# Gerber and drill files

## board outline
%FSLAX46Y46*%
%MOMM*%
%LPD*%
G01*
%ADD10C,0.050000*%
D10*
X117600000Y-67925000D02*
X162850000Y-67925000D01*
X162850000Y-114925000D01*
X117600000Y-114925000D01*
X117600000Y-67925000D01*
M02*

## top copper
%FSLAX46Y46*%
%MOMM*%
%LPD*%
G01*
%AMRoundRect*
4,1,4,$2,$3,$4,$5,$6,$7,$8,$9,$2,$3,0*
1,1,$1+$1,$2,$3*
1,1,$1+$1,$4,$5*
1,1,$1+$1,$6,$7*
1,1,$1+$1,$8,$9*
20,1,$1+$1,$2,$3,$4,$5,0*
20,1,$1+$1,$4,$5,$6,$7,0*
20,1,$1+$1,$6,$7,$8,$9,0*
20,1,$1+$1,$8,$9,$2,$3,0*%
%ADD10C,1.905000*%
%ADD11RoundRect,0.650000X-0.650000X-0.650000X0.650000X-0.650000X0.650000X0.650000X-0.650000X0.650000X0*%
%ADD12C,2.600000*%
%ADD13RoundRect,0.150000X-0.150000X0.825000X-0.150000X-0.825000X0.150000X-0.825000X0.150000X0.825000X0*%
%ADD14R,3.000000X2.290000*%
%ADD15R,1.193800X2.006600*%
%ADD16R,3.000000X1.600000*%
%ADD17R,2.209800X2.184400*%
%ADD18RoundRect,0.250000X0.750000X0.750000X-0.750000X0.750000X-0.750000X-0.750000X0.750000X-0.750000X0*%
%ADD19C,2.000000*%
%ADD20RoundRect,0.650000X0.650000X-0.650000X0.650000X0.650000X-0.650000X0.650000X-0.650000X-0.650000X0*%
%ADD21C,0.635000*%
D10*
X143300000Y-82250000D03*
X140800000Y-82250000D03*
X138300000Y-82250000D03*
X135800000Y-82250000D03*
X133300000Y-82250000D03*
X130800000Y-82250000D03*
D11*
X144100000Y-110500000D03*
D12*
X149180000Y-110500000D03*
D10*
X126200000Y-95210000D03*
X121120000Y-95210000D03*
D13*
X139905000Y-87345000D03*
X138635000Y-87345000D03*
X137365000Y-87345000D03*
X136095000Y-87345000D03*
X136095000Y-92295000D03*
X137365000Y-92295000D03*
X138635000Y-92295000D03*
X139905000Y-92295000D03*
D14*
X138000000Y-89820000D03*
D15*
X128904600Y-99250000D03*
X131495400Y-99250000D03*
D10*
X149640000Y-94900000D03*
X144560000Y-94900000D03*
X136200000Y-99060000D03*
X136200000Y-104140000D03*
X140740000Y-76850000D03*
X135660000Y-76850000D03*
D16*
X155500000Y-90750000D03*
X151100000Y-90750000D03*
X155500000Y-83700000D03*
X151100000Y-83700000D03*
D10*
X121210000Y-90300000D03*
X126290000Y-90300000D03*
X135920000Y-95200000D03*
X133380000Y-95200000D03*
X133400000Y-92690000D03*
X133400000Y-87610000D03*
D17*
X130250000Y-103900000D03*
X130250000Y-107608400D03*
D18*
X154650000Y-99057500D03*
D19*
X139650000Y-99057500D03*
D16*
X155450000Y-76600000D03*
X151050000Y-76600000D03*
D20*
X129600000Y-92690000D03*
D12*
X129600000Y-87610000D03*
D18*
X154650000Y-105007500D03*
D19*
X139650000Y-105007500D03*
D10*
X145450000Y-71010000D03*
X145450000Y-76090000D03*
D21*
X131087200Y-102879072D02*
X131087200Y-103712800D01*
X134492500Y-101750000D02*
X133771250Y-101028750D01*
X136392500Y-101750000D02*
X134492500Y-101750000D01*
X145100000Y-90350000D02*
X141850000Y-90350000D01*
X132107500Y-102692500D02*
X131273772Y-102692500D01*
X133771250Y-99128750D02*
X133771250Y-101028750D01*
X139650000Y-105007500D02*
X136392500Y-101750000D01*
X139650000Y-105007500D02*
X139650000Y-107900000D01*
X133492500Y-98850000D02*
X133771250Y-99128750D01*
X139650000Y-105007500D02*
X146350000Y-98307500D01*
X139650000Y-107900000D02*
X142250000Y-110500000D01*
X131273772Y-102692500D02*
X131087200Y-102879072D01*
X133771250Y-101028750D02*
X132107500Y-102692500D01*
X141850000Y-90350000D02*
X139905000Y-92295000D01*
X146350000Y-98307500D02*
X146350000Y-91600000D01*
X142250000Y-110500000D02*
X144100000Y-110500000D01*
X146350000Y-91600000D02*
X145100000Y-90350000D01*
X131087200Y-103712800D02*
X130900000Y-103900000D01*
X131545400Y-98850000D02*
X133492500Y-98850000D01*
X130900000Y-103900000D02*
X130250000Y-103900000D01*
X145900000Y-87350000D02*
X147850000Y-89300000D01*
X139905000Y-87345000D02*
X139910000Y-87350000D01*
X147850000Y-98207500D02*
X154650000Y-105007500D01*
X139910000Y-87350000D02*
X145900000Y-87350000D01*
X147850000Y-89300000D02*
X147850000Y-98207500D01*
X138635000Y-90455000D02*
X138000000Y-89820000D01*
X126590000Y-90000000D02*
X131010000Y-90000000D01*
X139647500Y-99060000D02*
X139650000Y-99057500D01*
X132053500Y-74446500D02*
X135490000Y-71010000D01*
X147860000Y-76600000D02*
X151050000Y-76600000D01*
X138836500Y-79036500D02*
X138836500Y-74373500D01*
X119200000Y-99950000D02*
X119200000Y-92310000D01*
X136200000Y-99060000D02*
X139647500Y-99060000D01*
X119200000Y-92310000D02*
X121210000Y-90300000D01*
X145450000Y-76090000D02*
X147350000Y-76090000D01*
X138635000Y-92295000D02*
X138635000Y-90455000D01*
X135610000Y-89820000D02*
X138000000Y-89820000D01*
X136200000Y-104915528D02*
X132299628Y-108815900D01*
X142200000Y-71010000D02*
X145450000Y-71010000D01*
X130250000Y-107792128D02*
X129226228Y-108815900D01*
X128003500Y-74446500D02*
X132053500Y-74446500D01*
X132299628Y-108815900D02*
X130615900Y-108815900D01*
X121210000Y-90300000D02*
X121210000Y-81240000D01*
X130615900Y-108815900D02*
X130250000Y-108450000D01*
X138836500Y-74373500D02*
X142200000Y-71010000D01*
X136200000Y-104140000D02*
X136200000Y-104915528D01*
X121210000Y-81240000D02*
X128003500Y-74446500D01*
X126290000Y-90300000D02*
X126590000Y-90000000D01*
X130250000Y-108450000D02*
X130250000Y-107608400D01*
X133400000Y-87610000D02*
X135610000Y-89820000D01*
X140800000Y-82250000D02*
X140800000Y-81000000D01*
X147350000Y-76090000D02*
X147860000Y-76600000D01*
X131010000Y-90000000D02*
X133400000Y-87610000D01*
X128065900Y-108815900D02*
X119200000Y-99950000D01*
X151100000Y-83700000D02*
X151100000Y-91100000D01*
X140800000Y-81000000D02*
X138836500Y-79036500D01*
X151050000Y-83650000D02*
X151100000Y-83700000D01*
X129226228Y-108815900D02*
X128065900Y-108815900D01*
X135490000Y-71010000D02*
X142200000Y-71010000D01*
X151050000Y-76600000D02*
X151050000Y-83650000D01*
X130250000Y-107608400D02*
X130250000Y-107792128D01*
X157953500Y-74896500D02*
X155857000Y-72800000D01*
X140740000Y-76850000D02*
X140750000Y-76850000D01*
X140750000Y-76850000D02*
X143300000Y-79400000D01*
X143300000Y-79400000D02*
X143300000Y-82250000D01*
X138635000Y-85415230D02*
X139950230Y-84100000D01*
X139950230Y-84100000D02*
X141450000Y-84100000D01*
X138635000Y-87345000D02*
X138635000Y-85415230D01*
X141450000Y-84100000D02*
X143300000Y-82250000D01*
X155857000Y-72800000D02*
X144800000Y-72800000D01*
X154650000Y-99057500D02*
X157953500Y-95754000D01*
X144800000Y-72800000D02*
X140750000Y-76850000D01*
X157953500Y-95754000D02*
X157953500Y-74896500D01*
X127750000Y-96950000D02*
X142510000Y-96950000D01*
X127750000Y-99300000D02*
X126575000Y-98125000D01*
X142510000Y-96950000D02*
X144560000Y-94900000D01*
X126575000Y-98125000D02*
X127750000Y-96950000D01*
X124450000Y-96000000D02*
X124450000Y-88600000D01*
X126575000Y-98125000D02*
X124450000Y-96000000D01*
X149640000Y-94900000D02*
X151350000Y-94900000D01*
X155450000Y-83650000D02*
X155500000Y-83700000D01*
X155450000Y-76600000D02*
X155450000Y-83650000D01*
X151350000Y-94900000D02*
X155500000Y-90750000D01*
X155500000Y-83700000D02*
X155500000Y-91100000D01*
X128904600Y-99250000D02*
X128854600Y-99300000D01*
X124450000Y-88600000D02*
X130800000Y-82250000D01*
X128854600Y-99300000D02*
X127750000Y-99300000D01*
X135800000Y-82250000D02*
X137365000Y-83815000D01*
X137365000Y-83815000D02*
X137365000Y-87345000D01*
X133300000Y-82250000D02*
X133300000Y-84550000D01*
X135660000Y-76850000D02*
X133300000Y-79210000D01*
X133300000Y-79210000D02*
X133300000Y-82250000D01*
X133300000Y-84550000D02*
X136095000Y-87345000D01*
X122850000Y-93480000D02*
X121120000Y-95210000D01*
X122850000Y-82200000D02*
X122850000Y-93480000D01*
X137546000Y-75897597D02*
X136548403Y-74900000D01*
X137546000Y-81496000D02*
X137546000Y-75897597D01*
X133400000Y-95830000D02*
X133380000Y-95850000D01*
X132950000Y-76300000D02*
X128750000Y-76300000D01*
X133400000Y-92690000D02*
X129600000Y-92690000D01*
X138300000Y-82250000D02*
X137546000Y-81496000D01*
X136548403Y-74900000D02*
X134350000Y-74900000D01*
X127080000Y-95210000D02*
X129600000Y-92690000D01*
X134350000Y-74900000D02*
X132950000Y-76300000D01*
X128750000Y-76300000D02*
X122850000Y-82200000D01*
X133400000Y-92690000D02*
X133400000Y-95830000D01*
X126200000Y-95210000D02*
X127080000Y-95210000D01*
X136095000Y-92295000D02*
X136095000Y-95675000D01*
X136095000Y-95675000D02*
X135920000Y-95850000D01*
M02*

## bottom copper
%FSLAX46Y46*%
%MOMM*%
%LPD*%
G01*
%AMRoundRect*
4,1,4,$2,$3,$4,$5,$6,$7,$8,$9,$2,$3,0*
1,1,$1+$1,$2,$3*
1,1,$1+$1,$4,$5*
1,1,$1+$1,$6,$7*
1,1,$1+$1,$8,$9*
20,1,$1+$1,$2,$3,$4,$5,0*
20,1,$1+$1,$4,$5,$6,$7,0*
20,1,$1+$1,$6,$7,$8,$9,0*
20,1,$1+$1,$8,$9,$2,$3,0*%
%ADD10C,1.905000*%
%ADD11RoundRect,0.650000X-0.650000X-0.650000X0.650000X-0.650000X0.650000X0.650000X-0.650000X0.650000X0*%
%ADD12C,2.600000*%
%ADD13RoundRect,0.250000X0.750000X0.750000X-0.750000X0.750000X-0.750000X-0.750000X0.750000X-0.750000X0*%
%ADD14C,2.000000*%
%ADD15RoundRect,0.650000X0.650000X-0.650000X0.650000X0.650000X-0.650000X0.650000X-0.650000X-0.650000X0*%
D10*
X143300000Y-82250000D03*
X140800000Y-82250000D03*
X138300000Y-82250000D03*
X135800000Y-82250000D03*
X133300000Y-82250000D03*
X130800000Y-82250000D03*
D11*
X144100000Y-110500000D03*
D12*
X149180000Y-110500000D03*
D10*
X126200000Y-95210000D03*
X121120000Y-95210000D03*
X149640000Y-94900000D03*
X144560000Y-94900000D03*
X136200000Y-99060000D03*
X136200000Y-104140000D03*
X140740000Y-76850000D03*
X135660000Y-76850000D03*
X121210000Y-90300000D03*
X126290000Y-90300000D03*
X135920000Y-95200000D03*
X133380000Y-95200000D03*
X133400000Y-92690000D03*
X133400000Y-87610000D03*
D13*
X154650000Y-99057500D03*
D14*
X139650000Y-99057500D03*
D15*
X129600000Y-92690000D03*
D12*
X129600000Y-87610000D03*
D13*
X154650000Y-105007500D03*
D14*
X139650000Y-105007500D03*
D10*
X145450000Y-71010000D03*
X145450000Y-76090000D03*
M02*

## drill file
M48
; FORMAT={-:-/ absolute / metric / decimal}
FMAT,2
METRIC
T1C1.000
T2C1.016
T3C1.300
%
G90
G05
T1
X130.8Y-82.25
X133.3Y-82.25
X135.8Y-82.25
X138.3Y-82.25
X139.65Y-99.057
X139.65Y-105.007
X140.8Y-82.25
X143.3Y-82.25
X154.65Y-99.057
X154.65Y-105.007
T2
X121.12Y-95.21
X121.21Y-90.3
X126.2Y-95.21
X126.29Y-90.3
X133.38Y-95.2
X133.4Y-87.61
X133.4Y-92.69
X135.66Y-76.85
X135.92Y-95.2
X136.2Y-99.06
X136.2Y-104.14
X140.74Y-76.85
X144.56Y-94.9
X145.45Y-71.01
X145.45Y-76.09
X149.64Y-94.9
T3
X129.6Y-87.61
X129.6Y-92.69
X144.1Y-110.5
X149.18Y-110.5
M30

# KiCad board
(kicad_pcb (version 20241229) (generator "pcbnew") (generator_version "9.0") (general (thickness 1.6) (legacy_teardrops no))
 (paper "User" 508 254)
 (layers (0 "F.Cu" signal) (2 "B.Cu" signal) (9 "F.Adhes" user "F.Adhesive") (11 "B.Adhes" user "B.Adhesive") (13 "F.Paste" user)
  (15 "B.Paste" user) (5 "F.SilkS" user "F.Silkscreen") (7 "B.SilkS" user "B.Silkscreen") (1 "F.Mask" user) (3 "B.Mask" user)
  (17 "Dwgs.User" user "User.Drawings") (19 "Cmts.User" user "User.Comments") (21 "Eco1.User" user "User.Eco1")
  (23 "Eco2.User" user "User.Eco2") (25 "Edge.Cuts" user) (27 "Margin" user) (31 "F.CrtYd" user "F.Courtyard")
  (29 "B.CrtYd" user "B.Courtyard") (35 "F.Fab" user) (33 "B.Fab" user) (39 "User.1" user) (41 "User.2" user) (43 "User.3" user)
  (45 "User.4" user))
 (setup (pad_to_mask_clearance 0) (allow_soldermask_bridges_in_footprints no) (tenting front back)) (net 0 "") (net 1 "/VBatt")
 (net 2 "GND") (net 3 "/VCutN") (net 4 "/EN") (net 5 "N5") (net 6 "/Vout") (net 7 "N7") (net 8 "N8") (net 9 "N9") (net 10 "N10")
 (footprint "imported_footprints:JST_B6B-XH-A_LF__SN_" (layer "F.Cu") (at 137.05 81.725)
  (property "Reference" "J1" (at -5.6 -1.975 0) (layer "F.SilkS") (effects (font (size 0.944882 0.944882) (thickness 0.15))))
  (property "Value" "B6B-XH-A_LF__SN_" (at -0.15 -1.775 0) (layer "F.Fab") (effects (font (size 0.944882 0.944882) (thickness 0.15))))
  (pad "1" thru_hole circle (at 6.25 0.525) (size 1.905 1.905) (drill 1) (layers "*.Cu" "*.Mask") (remove_unused_layers no) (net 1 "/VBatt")
   (solder_mask_margin 0.102))
  (pad "2" thru_hole circle (at 3.75 0.525) (size 1.905 1.905) (drill 1) (layers "*.Cu" "*.Mask") (remove_unused_layers no) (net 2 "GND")
   (solder_mask_margin 0.102))
  (pad "3" thru_hole circle (at 1.25 0.525) (size 1.905 1.905) (drill 1) (layers "*.Cu" "*.Mask") (remove_unused_layers no) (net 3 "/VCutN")
   (solder_mask_margin 0.102))
  (pad "4" thru_hole circle (at -1.25 0.525) (size 1.905 1.905) (drill 1) (layers "*.Cu" "*.Mask") (remove_unused_layers no) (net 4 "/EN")
   (solder_mask_margin 0.102))
  (pad "5" thru_hole circle (at -3.75 0.525) (size 1.905 1.905) (drill 1) (layers "*.Cu" "*.Mask") (remove_unused_layers no) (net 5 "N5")
   (solder_mask_margin 0.102))
  (pad "6" thru_hole circle (at -6.25 0.525) (size 1.905 1.905) (drill 1) (layers "*.Cu" "*.Mask") (remove_unused_layers no) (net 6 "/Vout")
   (solder_mask_margin 0.102)))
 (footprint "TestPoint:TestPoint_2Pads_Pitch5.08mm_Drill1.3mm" (layer "F.Cu") (at 144.1 110.5)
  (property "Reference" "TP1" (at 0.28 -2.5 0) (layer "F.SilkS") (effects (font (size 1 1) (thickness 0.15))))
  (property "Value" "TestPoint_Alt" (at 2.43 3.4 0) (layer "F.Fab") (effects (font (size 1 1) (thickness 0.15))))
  (pad "1" thru_hole roundrect (at 0 0) (size 2.6 2.6) (drill 1.3) (layers "*.Cu" "*.Mask") (remove_unused_layers no)
   (roundrect_rratio 0.25) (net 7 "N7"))
  (pad "2" thru_hole circle (at 5.08 0) (size 2.6 2.6) (drill 1.3) (layers "*.Cu" "*.Mask") (remove_unused_layers no)))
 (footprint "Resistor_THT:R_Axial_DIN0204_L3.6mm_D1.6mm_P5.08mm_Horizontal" (layer "F.Cu") (at 126.2 95.21 180)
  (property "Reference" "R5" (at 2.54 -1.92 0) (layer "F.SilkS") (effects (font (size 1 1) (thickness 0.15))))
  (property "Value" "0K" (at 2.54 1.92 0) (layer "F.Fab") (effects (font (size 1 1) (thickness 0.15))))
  (pad "1" thru_hole circle (at 0 0 180) (size 1.905 1.905) (drill 1.016) (layers "*.Cu" "*.Mask") (remove_unused_layers no)
   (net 3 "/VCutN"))
  (pad "2" thru_hole circle (at 5.08 0 180) (size 1.905 1.905) (drill 1.016) (layers "*.Cu" "*.Mask") (remove_unused_layers no)
   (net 3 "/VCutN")))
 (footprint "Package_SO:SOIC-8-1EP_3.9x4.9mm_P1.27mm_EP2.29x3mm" (layer "F.Cu") (at 138 89.82 -90)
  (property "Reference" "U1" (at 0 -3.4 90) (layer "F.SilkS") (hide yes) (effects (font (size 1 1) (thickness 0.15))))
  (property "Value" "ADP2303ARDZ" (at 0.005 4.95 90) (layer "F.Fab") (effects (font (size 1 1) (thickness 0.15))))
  (pad "" smd roundrect (at -0.57 -0.75 270) (size 0.92 1.21) (layers "F.Paste") (roundrect_rratio 0.25))
  (pad "" smd roundrect (at -0.57 0.75 270) (size 0.92 1.21) (layers "F.Paste") (roundrect_rratio 0.25))
  (pad "" smd roundrect (at 0.57 -0.75 270) (size 0.92 1.21) (layers "F.Paste") (roundrect_rratio 0.25))
  (pad "" smd roundrect (at 0.57 0.75 270) (size 0.92 1.21) (layers "F.Paste") (roundrect_rratio 0.25))
  (pad "1" smd roundrect (at -2.475 -1.905 270) (size 1.95 0.6) (layers "F.Cu" "F.Mask" "F.Paste") (roundrect_rratio 0.25) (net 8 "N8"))
  (pad "2" smd roundrect (at -2.475 -0.635 270) (size 1.95 0.6) (layers "F.Cu" "F.Mask" "F.Paste") (roundrect_rratio 0.25) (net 1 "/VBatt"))
  (pad "3" smd roundrect (at -2.475 0.635 270) (size 1.95 0.6) (layers "F.Cu" "F.Mask" "F.Paste") (roundrect_rratio 0.25) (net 4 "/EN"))
  (pad "4" smd roundrect (at -2.475 1.905 270) (size 1.95 0.6) (layers "F.Cu" "F.Mask" "F.Paste") (roundrect_rratio 0.25) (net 5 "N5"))
  (pad "5" smd roundrect (at 2.475 1.905 270) (size 1.95 0.6) (layers "F.Cu" "F.Mask" "F.Paste") (roundrect_rratio 0.25) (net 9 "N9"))
  (pad "6" smd roundrect (at 2.475 0.635 270) (size 1.95 0.6) (layers "F.Cu" "F.Mask" "F.Paste") (roundrect_rratio 0.25) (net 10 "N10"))
  (pad "7" smd roundrect (at 2.475 -0.635 270) (size 1.95 0.6) (layers "F.Cu" "F.Mask" "F.Paste") (roundrect_rratio 0.25) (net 2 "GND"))
  (pad "8" smd roundrect (at 2.475 -1.905 270) (size 1.95 0.6) (layers "F.Cu" "F.Mask" "F.Paste") (roundrect_rratio 0.25) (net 7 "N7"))
  (pad "9" smd rect (at 0 0 270) (size 2.29 3) (layers "F.Cu" "F.Mask") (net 2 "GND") (zone_connect 2)))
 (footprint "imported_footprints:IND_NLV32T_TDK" (layer "F.Cu") (at 130.2 99.25)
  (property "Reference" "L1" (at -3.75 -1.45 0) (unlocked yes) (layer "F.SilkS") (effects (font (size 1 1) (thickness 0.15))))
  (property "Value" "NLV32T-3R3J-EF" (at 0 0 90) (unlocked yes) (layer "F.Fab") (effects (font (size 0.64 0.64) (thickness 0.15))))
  (pad "1" smd rect (at -1.2954 0) (size 1.1938 2.0066) (layers "F.Cu" "F.Mask" "F.Paste") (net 6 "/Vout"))
  (pad "2" smd rect (at 1.2954 0) (size 1.1938 2.0066) (layers "F.Cu" "F.Mask" "F.Paste") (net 7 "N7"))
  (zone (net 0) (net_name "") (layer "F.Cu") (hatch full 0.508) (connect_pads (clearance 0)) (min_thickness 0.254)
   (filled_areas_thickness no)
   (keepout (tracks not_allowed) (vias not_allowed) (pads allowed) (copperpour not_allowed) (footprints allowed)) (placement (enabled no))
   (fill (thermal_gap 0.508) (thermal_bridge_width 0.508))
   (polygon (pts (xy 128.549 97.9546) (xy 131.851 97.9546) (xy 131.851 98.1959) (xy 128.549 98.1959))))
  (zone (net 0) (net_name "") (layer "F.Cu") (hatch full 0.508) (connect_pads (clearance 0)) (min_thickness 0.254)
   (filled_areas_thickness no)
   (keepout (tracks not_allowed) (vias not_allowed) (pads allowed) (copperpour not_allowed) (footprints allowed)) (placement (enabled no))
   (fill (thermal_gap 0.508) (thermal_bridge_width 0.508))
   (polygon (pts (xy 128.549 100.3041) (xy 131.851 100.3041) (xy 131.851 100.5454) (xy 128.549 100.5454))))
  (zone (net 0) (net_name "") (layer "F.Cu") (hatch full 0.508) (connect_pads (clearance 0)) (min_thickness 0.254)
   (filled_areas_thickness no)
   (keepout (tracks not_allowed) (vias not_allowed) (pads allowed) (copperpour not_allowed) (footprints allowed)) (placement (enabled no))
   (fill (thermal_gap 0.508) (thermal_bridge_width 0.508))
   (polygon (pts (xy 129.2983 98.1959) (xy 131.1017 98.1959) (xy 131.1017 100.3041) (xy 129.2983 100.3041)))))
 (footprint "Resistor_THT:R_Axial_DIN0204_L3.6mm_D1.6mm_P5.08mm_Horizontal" (layer "F.Cu") (at 149.64 94.9 180)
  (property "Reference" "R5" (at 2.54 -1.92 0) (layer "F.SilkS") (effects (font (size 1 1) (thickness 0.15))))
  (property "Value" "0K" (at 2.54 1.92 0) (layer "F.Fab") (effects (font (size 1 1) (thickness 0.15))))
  (pad "1" thru_hole circle (at 0 0 180) (size 1.905 1.905) (drill 1.016) (layers "*.Cu" "*.Mask") (remove_unused_layers no) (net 6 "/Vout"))
  (pad "2" thru_hole circle (at 5.08 0 180) (size 1.905 1.905) (drill 1.016) (layers "*.Cu" "*.Mask") (remove_unused_layers no)
   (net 6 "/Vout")))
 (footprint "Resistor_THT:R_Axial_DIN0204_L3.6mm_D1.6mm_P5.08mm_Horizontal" (layer "F.Cu") (at 136.2 99.06 -90)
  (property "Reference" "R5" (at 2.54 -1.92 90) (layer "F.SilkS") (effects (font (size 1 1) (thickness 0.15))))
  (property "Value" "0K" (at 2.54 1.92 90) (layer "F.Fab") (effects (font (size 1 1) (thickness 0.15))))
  (pad "1" thru_hole circle (at 0 0 270) (size 1.905 1.905) (drill 1.016) (layers "*.Cu" "*.Mask") (remove_unused_layers no) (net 2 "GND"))
  (pad "2" thru_hole circle (at 5.08 0 270) (size 1.905 1.905) (drill 1.016) (layers "*.Cu" "*.Mask") (remove_unused_layers no)
   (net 2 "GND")))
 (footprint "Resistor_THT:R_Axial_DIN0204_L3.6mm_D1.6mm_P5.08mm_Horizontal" (layer "F.Cu") (at 140.74 76.85 180)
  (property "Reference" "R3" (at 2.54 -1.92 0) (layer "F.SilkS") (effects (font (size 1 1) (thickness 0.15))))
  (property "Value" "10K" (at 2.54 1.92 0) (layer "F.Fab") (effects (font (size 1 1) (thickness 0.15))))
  (pad "1" thru_hole circle (at 0 0 180) (size 1.905 1.905) (drill 1.016) (layers "*.Cu" "*.Mask") (remove_unused_layers no)
   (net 1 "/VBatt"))
  (pad "2" thru_hole circle (at 5.08 0 180) (size 1.905 1.905) (drill 1.016) (layers "*.Cu" "*.Mask") (remove_unused_layers no) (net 5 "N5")))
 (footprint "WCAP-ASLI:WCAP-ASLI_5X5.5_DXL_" (layer "F.Cu") (at 153.3 90.75)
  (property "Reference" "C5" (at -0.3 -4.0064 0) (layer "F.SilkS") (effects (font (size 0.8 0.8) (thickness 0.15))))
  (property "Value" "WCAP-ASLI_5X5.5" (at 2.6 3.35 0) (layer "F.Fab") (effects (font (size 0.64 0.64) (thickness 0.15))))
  (pad "1" smd rect (at 2.2 0) (size 3 1.6) (layers "F.Cu" "F.Mask" "F.Paste") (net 6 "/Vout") (solder_mask_margin 0.102))
  (pad "2" smd rect (at -2.2 0) (size 3 1.6) (layers "F.Cu" "F.Mask" "F.Paste") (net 2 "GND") (solder_mask_margin 0.102)))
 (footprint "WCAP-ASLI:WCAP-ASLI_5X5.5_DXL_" (layer "F.Cu") (at 153.3 83.7)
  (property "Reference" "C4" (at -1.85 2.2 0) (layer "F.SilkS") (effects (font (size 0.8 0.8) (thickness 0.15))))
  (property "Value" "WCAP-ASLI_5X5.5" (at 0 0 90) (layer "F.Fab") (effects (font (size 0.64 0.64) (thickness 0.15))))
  (pad "1" smd rect (at 2.2 0) (size 3 1.6) (layers "F.Cu" "F.Mask" "F.Paste") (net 6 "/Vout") (solder_mask_margin 0.102))
  (pad "2" smd rect (at -2.2 0) (size 3 1.6) (layers "F.Cu" "F.Mask" "F.Paste") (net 2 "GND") (solder_mask_margin 0.102)))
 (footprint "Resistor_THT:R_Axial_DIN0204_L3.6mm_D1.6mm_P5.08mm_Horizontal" (layer "F.Cu") (at 121.21 90.3)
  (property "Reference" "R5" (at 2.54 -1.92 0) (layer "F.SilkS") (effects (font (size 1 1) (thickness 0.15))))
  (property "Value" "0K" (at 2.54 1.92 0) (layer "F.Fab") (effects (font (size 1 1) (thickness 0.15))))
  (pad "1" thru_hole circle (at 0 0) (size 1.905 1.905) (drill 1.016) (layers "*.Cu" "*.Mask") (remove_unused_layers no) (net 2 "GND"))
  (pad "2" thru_hole circle (at 5.08 0) (size 1.905 1.905) (drill 1.016) (layers "*.Cu" "*.Mask") (remove_unused_layers no) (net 2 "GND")))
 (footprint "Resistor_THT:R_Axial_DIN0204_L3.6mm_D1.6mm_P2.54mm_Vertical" (layer "F.Cu") (at 135.92 95.2 180)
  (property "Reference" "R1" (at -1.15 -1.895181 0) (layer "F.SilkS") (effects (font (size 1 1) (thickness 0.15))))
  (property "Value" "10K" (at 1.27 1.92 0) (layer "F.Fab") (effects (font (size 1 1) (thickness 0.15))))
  (pad "1" thru_hole circle (at 0 0 180) (size 1.905 1.905) (drill 1.016) (layers "*.Cu" "*.Mask") (remove_unused_layers no) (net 9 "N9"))
  (pad "2" thru_hole circle (at 2.54 0 180) (size 1.905 1.905) (drill 1.016) (layers "*.Cu" "*.Mask") (remove_unused_layers no)
   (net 3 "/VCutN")))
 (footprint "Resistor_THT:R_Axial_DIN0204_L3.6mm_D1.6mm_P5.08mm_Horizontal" (layer "F.Cu") (at 133.4 92.69 90)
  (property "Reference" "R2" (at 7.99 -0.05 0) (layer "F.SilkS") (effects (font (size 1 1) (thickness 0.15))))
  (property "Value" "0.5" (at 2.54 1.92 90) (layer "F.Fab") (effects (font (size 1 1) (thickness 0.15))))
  (pad "1" thru_hole circle (at 0 0 90) (size 1.905 1.905) (drill 1.016) (layers "*.Cu" "*.Mask") (remove_unused_layers no) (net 3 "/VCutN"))
  (pad "2" thru_hole circle (at 5.08 0 90) (size 1.905 1.905) (drill 1.016) (layers "*.Cu" "*.Mask") (remove_unused_layers no) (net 2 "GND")))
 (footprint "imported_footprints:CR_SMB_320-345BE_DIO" (layer "F.Cu") (at 130.25 105.7542 -90)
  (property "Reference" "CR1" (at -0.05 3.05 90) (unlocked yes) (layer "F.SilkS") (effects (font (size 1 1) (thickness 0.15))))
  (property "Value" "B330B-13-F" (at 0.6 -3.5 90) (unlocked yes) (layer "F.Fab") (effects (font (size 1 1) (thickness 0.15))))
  (pad "1" smd rect (at -1.8542 0) (size 2.2098 2.1844) (layers "F.Cu" "F.Mask" "F.Paste") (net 7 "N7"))
  (pad "2" smd rect (at 1.8542 0) (size 2.2098 2.1844) (layers "F.Cu" "F.Mask" "F.Paste") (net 2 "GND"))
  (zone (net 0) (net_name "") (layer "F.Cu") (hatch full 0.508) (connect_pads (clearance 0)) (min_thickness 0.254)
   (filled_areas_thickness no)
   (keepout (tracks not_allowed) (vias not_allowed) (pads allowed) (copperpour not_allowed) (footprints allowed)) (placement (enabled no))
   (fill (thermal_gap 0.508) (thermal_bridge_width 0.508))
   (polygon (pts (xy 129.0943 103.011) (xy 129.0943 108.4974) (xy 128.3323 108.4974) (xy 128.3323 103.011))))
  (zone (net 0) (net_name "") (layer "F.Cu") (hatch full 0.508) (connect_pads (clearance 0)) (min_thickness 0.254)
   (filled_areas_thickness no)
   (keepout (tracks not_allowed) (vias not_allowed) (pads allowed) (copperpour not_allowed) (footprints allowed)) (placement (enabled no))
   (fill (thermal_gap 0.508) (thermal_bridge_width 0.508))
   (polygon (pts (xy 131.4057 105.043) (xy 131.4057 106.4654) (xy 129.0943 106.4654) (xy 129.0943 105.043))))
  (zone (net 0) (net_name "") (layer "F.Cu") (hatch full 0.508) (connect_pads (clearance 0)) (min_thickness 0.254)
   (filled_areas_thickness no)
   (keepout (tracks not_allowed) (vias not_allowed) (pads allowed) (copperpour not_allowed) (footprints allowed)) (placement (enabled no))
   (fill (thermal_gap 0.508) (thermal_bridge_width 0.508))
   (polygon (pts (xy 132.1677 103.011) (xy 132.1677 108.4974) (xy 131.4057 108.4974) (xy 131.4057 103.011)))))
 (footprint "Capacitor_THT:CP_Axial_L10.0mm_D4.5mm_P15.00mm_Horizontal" (layer "F.Cu") (at 154.65 99.0575 180)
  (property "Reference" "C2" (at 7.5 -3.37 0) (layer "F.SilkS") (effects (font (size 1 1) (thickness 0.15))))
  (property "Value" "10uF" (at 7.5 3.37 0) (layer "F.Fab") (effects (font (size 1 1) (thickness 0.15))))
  (pad "1" thru_hole roundrect (at 0 0 180) (size 2 2) (drill 1) (layers "*.Cu" "*.Mask") (remove_unused_layers no) (roundrect_rratio 0.125)
   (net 1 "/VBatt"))
  (pad "2" thru_hole circle (at 15 0 180) (size 2 2) (drill 1) (layers "*.Cu" "*.Mask") (remove_unused_layers no) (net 2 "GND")))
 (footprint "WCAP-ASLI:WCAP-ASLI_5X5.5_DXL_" (layer "F.Cu") (at 153.25 76.6)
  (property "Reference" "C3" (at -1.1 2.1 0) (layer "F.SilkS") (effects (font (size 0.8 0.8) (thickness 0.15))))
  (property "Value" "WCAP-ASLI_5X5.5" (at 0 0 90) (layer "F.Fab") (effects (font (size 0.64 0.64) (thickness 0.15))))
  (pad "1" smd rect (at 2.2 0) (size 3 1.6) (layers "F.Cu" "F.Mask" "F.Paste") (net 6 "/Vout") (solder_mask_margin 0.102))
  (pad "2" smd rect (at -2.2 0) (size 3 1.6) (layers "F.Cu" "F.Mask" "F.Paste") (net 2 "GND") (solder_mask_margin 0.102)))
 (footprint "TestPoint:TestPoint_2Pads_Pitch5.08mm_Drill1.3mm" (layer "F.Cu") (at 129.6 92.69 90)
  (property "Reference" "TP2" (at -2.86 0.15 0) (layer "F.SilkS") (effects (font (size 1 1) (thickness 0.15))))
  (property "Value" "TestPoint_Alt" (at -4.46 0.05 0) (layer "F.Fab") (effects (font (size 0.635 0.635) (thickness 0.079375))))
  (pad "1" thru_hole roundrect (at 0 0 90) (size 2.6 2.6) (drill 1.3) (layers "*.Cu" "*.Mask") (remove_unused_layers no)
   (roundrect_rratio 0.25) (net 3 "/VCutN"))
  (pad "2" thru_hole circle (at 5.08 0 90) (size 2.6 2.6) (drill 1.3) (layers "*.Cu" "*.Mask") (remove_unused_layers no)))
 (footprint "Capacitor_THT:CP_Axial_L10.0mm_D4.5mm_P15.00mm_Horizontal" (layer "F.Cu") (at 154.65 105.0075 180)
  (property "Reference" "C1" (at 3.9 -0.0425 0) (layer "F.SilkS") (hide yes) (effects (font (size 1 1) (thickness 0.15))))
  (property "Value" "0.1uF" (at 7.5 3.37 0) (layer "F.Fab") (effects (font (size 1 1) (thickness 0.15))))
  (pad "1" thru_hole roundrect (at 0 0 180) (size 2 2) (drill 1) (layers "*.Cu" "*.Mask") (remove_unused_layers no) (roundrect_rratio 0.125)
   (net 8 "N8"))
  (pad "2" thru_hole circle (at 15 0 180) (size 2 2) (drill 1) (layers "*.Cu" "*.Mask") (remove_unused_layers no) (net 7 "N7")))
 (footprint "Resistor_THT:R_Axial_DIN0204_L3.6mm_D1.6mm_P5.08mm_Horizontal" (layer "F.Cu") (at 145.45 71.01 -90)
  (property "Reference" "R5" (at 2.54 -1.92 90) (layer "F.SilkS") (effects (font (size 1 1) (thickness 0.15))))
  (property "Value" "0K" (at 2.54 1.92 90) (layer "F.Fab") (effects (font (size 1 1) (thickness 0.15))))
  (pad "1" thru_hole circle (at 0 0 270) (size 1.905 1.905) (drill 1.016) (layers "*.Cu" "*.Mask") (remove_unused_layers no) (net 2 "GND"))
  (pad "2" thru_hole circle (at 5.08 0 270) (size 1.905 1.905) (drill 1.016) (layers "*.Cu" "*.Mask") (remove_unused_layers no)
   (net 2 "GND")))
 (gr_rect (start 117.6 67.925) (end 162.85 114.925) (stroke (width 0.05) (type default)) (fill no) (layer "Edge.Cuts"))
 (segment (start 131.0872 102.879072) (end 131.0872 103.7128) (width 0.635) (layer "F.Cu") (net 7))
 (segment (start 134.4925 101.75) (end 133.77125 101.02875) (width 0.635) (layer "F.Cu") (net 7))
 (segment (start 136.3925 101.75) (end 134.4925 101.75) (width 0.635) (layer "F.Cu") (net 7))
 (segment (start 145.1 90.35) (end 141.85 90.35) (width 0.635) (layer "F.Cu") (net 7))
 (segment (start 132.1075 102.6925) (end 131.273772 102.6925) (width 0.635) (layer "F.Cu") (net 7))
 (segment (start 133.77125 99.12875) (end 133.77125 101.02875) (width 0.635) (layer "F.Cu") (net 7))
 (segment (start 139.65 105.0075) (end 136.3925 101.75) (width 0.635) (layer "F.Cu") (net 7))
 (segment (start 139.65 105.0075) (end 139.65 107.9) (width 0.635) (layer "F.Cu") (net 7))
 (segment (start 133.4925 98.85) (end 133.77125 99.12875) (width 0.635) (layer "F.Cu") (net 7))
 (segment (start 139.65 105.0075) (end 146.35 98.3075) (width 0.635) (layer "F.Cu") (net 7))
 (segment (start 139.65 107.9) (end 142.25 110.5) (width 0.635) (layer "F.Cu") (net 7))
 (segment (start 131.273772 102.6925) (end 131.0872 102.879072) (width 0.635) (layer "F.Cu") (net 7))
 (segment (start 133.77125 101.02875) (end 132.1075 102.6925) (width 0.635) (layer "F.Cu") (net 7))
 (segment (start 141.85 90.35) (end 139.905 92.295) (width 0.635) (layer "F.Cu") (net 7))
 (segment (start 146.35 98.3075) (end 146.35 91.6) (width 0.635) (layer "F.Cu") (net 7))
 (segment (start 142.25 110.5) (end 144.1 110.5) (width 0.635) (layer "F.Cu") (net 7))
 (segment (start 146.35 91.6) (end 145.1 90.35) (width 0.635) (layer "F.Cu") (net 7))
 (segment (start 131.0872 103.7128) (end 130.9 103.9) (width 0.635) (layer "F.Cu") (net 7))
 (segment (start 131.5454 98.85) (end 133.4925 98.85) (width 0.635) (layer "F.Cu") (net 7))
 (segment (start 130.9 103.9) (end 130.25 103.9) (width 0.635) (layer "F.Cu") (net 7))
 (segment (start 145.9 87.35) (end 147.85 89.3) (width 0.635) (layer "F.Cu") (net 8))
 (segment (start 139.905 87.345) (end 139.91 87.35) (width 0.635) (layer "F.Cu") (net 8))
 (segment (start 147.85 98.2075) (end 154.65 105.0075) (width 0.635) (layer "F.Cu") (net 8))
 (segment (start 139.91 87.35) (end 145.9 87.35) (width 0.635) (layer "F.Cu") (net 8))
 (segment (start 147.85 89.3) (end 147.85 98.2075) (width 0.635) (layer "F.Cu") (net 8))
 (segment (start 138.635 90.455) (end 138 89.82) (width 0.635) (layer "F.Cu") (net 2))
 (segment (start 126.59 90) (end 131.01 90) (width 0.635) (layer "F.Cu") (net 2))
 (segment (start 139.6475 99.06) (end 139.65 99.0575) (width 0.635) (layer "F.Cu") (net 2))
 (segment (start 132.0535 74.4465) (end 135.49 71.01) (width 0.635) (layer "F.Cu") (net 2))
 (segment (start 147.86 76.6) (end 151.05 76.6) (width 0.635) (layer "F.Cu") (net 2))
 (segment (start 138.8365 79.0365) (end 138.8365 74.3735) (width 0.635) (layer "F.Cu") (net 2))
 (segment (start 119.2 99.95) (end 119.2 92.31) (width 0.635) (layer "F.Cu") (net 2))
 (segment (start 136.2 99.06) (end 139.6475 99.06) (width 0.635) (layer "F.Cu") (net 2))
 (segment (start 119.2 92.31) (end 121.21 90.3) (width 0.635) (layer "F.Cu") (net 2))
 (segment (start 145.45 76.09) (end 147.35 76.09) (width 0.635) (layer "F.Cu") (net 2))
 (segment (start 138.635 92.295) (end 138.635 90.455) (width 0.635) (layer "F.Cu") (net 2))
 (segment (start 135.61 89.82) (end 138 89.82) (width 0.635) (layer "F.Cu") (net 2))
 (segment (start 136.2 104.915528) (end 132.299628 108.8159) (width 0.635) (layer "F.Cu") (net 2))
 (segment (start 142.2 71.01) (end 145.45 71.01) (width 0.635) (layer "F.Cu") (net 2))
 (segment (start 130.25 107.792128) (end 129.226228 108.8159) (width 0.635) (layer "F.Cu") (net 2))
 (segment (start 128.0035 74.4465) (end 132.0535 74.4465) (width 0.635) (layer "F.Cu") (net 2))
 (segment (start 132.299628 108.8159) (end 130.6159 108.8159) (width 0.635) (layer "F.Cu") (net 2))
 (segment (start 121.21 90.3) (end 121.21 81.24) (width 0.635) (layer "F.Cu") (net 2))
 (segment (start 130.6159 108.8159) (end 130.25 108.45) (width 0.635) (layer "F.Cu") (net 2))
 (segment (start 138.8365 74.3735) (end 142.2 71.01) (width 0.635) (layer "F.Cu") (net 2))
 (segment (start 136.2 104.14) (end 136.2 104.915528) (width 0.635) (layer "F.Cu") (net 2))
 (segment (start 121.21 81.24) (end 128.0035 74.4465) (width 0.635) (layer "F.Cu") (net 2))
 (segment (start 126.29 90.3) (end 126.59 90) (width 0.635) (layer "F.Cu") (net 2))
 (segment (start 130.25 108.45) (end 130.25 107.6084) (width 0.635) (layer "F.Cu") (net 2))
 (segment (start 133.4 87.61) (end 135.61 89.82) (width 0.635) (layer "F.Cu") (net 2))
 (segment (start 140.8 82.25) (end 140.8 81) (width 0.635) (layer "F.Cu") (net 2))
 (segment (start 147.35 76.09) (end 147.86 76.6) (width 0.635) (layer "F.Cu") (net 2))
 (segment (start 131.01 90) (end 133.4 87.61) (width 0.635) (layer "F.Cu") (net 2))
 (segment (start 128.0659 108.8159) (end 119.2 99.95) (width 0.635) (layer "F.Cu") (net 2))
 (segment (start 151.1 83.7) (end 151.1 91.1) (width 0.635) (layer "F.Cu") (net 2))
 (segment (start 140.8 81) (end 138.8365 79.0365) (width 0.635) (layer "F.Cu") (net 2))
 (segment (start 151.05 83.65) (end 151.1 83.7) (width 0.635) (layer "F.Cu") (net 2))
 (segment (start 129.226228 108.8159) (end 128.0659 108.8159) (width 0.635) (layer "F.Cu") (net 2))
 (segment (start 135.49 71.01) (end 142.2 71.01) (width 0.635) (layer "F.Cu") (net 2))
 (segment (start 151.05 76.6) (end 151.05 83.65) (width 0.635) (layer "F.Cu") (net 2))
 (segment (start 130.25 107.6084) (end 130.25 107.792128) (width 0.635) (layer "F.Cu") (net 2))
 (segment (start 157.9535 74.8965) (end 155.857 72.8) (width 0.635) (layer "F.Cu") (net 1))
 (segment (start 140.74 76.85) (end 140.75 76.85) (width 0.635) (layer "F.Cu") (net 1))
 (segment (start 140.75 76.85) (end 143.3 79.4) (width 0.635) (layer "F.Cu") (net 1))
 (segment (start 143.3 79.4) (end 143.3 82.25) (width 0.635) (layer "F.Cu") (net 1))
 (segment (start 138.635 85.41523) (end 139.95023 84.1) (width 0.635) (layer "F.Cu") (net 1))
 (segment (start 139.95023 84.1) (end 141.45 84.1) (width 0.635) (layer "F.Cu") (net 1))
 (segment (start 138.635 87.345) (end 138.635 85.41523) (width 0.635) (layer "F.Cu") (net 1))
 (segment (start 141.45 84.1) (end 143.3 82.25) (width 0.635) (layer "F.Cu") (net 1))
 (segment (start 155.857 72.8) (end 144.8 72.8) (width 0.635) (layer "F.Cu") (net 1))
 (segment (start 154.65 99.0575) (end 157.9535 95.754) (width 0.635) (layer "F.Cu") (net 1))
 (segment (start 144.8 72.8) (end 140.75 76.85) (width 0.635) (layer "F.Cu") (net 1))
 (segment (start 157.9535 95.754) (end 157.9535 74.8965) (width 0.635) (layer "F.Cu") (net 1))
 (segment (start 127.75 96.95) (end 142.51 96.95) (width 0.635) (layer "F.Cu") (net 6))
 (segment (start 127.75 99.3) (end 126.575 98.125) (width 0.635) (layer "F.Cu") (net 6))
 (segment (start 142.51 96.95) (end 144.56 94.9) (width 0.635) (layer "F.Cu") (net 6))
 (segment (start 126.575 98.125) (end 127.75 96.95) (width 0.635) (layer "F.Cu") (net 6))
 (segment (start 124.45 96) (end 124.45 88.6) (width 0.635) (layer "F.Cu") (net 6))
 (segment (start 126.575 98.125) (end 124.45 96) (width 0.635) (layer "F.Cu") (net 6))
 (segment (start 149.64 94.9) (end 151.35 94.9) (width 0.635) (layer "F.Cu") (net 6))
 (segment (start 155.45 83.65) (end 155.5 83.7) (width 0.635) (layer "F.Cu") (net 6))
 (segment (start 155.45 76.6) (end 155.45 83.65) (width 0.635) (layer "F.Cu") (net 6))
 (segment (start 151.35 94.9) (end 155.5 90.75) (width 0.635) (layer "F.Cu") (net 6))
 (segment (start 155.5 83.7) (end 155.5 91.1) (width 0.635) (layer "F.Cu") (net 6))
 (segment (start 128.9046 99.25) (end 128.8546 99.3) (width 0.635) (layer "F.Cu") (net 6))
 (segment (start 124.45 88.6) (end 130.8 82.25) (width 0.635) (layer "F.Cu") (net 6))
 (segment (start 128.8546 99.3) (end 127.75 99.3) (width 0.635) (layer "F.Cu") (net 6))
 (segment (start 135.8 82.25) (end 137.365 83.815) (width 0.635) (layer "F.Cu") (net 4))
 (segment (start 137.365 83.815) (end 137.365 87.345) (width 0.635) (layer "F.Cu") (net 4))
 (segment (start 133.3 82.25) (end 133.3 84.55) (width 0.635) (layer "F.Cu") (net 5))
 (segment (start 135.66 76.85) (end 133.3 79.21) (width 0.635) (layer "F.Cu") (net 5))
 (segment (start 133.3 79.21) (end 133.3 82.25) (width 0.635) (layer "F.Cu") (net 5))
 (segment (start 133.3 84.55) (end 136.095 87.345) (width 0.635) (layer "F.Cu") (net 5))
 (segment (start 122.85 93.48) (end 121.12 95.21) (width 0.635) (layer "F.Cu") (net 3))
 (segment (start 122.85 82.2) (end 122.85 93.48) (width 0.635) (layer "F.Cu") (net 3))
 (segment (start 137.546 75.897597) (end 136.548403 74.9) (width 0.635) (layer "F.Cu") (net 3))
 (segment (start 137.546 81.496) (end 137.546 75.897597) (width 0.635) (layer "F.Cu") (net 3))
 (segment (start 133.4 95.83) (end 133.38 95.85) (width 0.635) (layer "F.Cu") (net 3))
 (segment (start 132.95 76.3) (end 128.75 76.3) (width 0.635) (layer "F.Cu") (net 3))
 (segment (start 133.4 92.69) (end 129.6 92.69) (width 0.635) (layer "F.Cu") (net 3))
 (segment (start 138.3 82.25) (end 137.546 81.496) (width 0.635) (layer "F.Cu") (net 3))
 (segment (start 136.548403 74.9) (end 134.35 74.9) (width 0.635) (layer "F.Cu") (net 3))
 (segment (start 127.08 95.21) (end 129.6 92.69) (width 0.635) (layer "F.Cu") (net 3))
 (segment (start 134.35 74.9) (end 132.95 76.3) (width 0.635) (layer "F.Cu") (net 3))
 (segment (start 128.75 76.3) (end 122.85 82.2) (width 0.635) (layer "F.Cu") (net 3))
 (segment (start 133.4 92.69) (end 133.4 95.83) (width 0.635) (layer "F.Cu") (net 3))
 (segment (start 126.2 95.21) (end 127.08 95.21) (width 0.635) (layer "F.Cu") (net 3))
 (segment (start 136.095 92.295) (end 136.095 95.675) (width 0.635) (layer "F.Cu") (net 9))
 (segment (start 136.095 95.675) (end 135.92 95.85) (width 0.635) (layer "F.Cu") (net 9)))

